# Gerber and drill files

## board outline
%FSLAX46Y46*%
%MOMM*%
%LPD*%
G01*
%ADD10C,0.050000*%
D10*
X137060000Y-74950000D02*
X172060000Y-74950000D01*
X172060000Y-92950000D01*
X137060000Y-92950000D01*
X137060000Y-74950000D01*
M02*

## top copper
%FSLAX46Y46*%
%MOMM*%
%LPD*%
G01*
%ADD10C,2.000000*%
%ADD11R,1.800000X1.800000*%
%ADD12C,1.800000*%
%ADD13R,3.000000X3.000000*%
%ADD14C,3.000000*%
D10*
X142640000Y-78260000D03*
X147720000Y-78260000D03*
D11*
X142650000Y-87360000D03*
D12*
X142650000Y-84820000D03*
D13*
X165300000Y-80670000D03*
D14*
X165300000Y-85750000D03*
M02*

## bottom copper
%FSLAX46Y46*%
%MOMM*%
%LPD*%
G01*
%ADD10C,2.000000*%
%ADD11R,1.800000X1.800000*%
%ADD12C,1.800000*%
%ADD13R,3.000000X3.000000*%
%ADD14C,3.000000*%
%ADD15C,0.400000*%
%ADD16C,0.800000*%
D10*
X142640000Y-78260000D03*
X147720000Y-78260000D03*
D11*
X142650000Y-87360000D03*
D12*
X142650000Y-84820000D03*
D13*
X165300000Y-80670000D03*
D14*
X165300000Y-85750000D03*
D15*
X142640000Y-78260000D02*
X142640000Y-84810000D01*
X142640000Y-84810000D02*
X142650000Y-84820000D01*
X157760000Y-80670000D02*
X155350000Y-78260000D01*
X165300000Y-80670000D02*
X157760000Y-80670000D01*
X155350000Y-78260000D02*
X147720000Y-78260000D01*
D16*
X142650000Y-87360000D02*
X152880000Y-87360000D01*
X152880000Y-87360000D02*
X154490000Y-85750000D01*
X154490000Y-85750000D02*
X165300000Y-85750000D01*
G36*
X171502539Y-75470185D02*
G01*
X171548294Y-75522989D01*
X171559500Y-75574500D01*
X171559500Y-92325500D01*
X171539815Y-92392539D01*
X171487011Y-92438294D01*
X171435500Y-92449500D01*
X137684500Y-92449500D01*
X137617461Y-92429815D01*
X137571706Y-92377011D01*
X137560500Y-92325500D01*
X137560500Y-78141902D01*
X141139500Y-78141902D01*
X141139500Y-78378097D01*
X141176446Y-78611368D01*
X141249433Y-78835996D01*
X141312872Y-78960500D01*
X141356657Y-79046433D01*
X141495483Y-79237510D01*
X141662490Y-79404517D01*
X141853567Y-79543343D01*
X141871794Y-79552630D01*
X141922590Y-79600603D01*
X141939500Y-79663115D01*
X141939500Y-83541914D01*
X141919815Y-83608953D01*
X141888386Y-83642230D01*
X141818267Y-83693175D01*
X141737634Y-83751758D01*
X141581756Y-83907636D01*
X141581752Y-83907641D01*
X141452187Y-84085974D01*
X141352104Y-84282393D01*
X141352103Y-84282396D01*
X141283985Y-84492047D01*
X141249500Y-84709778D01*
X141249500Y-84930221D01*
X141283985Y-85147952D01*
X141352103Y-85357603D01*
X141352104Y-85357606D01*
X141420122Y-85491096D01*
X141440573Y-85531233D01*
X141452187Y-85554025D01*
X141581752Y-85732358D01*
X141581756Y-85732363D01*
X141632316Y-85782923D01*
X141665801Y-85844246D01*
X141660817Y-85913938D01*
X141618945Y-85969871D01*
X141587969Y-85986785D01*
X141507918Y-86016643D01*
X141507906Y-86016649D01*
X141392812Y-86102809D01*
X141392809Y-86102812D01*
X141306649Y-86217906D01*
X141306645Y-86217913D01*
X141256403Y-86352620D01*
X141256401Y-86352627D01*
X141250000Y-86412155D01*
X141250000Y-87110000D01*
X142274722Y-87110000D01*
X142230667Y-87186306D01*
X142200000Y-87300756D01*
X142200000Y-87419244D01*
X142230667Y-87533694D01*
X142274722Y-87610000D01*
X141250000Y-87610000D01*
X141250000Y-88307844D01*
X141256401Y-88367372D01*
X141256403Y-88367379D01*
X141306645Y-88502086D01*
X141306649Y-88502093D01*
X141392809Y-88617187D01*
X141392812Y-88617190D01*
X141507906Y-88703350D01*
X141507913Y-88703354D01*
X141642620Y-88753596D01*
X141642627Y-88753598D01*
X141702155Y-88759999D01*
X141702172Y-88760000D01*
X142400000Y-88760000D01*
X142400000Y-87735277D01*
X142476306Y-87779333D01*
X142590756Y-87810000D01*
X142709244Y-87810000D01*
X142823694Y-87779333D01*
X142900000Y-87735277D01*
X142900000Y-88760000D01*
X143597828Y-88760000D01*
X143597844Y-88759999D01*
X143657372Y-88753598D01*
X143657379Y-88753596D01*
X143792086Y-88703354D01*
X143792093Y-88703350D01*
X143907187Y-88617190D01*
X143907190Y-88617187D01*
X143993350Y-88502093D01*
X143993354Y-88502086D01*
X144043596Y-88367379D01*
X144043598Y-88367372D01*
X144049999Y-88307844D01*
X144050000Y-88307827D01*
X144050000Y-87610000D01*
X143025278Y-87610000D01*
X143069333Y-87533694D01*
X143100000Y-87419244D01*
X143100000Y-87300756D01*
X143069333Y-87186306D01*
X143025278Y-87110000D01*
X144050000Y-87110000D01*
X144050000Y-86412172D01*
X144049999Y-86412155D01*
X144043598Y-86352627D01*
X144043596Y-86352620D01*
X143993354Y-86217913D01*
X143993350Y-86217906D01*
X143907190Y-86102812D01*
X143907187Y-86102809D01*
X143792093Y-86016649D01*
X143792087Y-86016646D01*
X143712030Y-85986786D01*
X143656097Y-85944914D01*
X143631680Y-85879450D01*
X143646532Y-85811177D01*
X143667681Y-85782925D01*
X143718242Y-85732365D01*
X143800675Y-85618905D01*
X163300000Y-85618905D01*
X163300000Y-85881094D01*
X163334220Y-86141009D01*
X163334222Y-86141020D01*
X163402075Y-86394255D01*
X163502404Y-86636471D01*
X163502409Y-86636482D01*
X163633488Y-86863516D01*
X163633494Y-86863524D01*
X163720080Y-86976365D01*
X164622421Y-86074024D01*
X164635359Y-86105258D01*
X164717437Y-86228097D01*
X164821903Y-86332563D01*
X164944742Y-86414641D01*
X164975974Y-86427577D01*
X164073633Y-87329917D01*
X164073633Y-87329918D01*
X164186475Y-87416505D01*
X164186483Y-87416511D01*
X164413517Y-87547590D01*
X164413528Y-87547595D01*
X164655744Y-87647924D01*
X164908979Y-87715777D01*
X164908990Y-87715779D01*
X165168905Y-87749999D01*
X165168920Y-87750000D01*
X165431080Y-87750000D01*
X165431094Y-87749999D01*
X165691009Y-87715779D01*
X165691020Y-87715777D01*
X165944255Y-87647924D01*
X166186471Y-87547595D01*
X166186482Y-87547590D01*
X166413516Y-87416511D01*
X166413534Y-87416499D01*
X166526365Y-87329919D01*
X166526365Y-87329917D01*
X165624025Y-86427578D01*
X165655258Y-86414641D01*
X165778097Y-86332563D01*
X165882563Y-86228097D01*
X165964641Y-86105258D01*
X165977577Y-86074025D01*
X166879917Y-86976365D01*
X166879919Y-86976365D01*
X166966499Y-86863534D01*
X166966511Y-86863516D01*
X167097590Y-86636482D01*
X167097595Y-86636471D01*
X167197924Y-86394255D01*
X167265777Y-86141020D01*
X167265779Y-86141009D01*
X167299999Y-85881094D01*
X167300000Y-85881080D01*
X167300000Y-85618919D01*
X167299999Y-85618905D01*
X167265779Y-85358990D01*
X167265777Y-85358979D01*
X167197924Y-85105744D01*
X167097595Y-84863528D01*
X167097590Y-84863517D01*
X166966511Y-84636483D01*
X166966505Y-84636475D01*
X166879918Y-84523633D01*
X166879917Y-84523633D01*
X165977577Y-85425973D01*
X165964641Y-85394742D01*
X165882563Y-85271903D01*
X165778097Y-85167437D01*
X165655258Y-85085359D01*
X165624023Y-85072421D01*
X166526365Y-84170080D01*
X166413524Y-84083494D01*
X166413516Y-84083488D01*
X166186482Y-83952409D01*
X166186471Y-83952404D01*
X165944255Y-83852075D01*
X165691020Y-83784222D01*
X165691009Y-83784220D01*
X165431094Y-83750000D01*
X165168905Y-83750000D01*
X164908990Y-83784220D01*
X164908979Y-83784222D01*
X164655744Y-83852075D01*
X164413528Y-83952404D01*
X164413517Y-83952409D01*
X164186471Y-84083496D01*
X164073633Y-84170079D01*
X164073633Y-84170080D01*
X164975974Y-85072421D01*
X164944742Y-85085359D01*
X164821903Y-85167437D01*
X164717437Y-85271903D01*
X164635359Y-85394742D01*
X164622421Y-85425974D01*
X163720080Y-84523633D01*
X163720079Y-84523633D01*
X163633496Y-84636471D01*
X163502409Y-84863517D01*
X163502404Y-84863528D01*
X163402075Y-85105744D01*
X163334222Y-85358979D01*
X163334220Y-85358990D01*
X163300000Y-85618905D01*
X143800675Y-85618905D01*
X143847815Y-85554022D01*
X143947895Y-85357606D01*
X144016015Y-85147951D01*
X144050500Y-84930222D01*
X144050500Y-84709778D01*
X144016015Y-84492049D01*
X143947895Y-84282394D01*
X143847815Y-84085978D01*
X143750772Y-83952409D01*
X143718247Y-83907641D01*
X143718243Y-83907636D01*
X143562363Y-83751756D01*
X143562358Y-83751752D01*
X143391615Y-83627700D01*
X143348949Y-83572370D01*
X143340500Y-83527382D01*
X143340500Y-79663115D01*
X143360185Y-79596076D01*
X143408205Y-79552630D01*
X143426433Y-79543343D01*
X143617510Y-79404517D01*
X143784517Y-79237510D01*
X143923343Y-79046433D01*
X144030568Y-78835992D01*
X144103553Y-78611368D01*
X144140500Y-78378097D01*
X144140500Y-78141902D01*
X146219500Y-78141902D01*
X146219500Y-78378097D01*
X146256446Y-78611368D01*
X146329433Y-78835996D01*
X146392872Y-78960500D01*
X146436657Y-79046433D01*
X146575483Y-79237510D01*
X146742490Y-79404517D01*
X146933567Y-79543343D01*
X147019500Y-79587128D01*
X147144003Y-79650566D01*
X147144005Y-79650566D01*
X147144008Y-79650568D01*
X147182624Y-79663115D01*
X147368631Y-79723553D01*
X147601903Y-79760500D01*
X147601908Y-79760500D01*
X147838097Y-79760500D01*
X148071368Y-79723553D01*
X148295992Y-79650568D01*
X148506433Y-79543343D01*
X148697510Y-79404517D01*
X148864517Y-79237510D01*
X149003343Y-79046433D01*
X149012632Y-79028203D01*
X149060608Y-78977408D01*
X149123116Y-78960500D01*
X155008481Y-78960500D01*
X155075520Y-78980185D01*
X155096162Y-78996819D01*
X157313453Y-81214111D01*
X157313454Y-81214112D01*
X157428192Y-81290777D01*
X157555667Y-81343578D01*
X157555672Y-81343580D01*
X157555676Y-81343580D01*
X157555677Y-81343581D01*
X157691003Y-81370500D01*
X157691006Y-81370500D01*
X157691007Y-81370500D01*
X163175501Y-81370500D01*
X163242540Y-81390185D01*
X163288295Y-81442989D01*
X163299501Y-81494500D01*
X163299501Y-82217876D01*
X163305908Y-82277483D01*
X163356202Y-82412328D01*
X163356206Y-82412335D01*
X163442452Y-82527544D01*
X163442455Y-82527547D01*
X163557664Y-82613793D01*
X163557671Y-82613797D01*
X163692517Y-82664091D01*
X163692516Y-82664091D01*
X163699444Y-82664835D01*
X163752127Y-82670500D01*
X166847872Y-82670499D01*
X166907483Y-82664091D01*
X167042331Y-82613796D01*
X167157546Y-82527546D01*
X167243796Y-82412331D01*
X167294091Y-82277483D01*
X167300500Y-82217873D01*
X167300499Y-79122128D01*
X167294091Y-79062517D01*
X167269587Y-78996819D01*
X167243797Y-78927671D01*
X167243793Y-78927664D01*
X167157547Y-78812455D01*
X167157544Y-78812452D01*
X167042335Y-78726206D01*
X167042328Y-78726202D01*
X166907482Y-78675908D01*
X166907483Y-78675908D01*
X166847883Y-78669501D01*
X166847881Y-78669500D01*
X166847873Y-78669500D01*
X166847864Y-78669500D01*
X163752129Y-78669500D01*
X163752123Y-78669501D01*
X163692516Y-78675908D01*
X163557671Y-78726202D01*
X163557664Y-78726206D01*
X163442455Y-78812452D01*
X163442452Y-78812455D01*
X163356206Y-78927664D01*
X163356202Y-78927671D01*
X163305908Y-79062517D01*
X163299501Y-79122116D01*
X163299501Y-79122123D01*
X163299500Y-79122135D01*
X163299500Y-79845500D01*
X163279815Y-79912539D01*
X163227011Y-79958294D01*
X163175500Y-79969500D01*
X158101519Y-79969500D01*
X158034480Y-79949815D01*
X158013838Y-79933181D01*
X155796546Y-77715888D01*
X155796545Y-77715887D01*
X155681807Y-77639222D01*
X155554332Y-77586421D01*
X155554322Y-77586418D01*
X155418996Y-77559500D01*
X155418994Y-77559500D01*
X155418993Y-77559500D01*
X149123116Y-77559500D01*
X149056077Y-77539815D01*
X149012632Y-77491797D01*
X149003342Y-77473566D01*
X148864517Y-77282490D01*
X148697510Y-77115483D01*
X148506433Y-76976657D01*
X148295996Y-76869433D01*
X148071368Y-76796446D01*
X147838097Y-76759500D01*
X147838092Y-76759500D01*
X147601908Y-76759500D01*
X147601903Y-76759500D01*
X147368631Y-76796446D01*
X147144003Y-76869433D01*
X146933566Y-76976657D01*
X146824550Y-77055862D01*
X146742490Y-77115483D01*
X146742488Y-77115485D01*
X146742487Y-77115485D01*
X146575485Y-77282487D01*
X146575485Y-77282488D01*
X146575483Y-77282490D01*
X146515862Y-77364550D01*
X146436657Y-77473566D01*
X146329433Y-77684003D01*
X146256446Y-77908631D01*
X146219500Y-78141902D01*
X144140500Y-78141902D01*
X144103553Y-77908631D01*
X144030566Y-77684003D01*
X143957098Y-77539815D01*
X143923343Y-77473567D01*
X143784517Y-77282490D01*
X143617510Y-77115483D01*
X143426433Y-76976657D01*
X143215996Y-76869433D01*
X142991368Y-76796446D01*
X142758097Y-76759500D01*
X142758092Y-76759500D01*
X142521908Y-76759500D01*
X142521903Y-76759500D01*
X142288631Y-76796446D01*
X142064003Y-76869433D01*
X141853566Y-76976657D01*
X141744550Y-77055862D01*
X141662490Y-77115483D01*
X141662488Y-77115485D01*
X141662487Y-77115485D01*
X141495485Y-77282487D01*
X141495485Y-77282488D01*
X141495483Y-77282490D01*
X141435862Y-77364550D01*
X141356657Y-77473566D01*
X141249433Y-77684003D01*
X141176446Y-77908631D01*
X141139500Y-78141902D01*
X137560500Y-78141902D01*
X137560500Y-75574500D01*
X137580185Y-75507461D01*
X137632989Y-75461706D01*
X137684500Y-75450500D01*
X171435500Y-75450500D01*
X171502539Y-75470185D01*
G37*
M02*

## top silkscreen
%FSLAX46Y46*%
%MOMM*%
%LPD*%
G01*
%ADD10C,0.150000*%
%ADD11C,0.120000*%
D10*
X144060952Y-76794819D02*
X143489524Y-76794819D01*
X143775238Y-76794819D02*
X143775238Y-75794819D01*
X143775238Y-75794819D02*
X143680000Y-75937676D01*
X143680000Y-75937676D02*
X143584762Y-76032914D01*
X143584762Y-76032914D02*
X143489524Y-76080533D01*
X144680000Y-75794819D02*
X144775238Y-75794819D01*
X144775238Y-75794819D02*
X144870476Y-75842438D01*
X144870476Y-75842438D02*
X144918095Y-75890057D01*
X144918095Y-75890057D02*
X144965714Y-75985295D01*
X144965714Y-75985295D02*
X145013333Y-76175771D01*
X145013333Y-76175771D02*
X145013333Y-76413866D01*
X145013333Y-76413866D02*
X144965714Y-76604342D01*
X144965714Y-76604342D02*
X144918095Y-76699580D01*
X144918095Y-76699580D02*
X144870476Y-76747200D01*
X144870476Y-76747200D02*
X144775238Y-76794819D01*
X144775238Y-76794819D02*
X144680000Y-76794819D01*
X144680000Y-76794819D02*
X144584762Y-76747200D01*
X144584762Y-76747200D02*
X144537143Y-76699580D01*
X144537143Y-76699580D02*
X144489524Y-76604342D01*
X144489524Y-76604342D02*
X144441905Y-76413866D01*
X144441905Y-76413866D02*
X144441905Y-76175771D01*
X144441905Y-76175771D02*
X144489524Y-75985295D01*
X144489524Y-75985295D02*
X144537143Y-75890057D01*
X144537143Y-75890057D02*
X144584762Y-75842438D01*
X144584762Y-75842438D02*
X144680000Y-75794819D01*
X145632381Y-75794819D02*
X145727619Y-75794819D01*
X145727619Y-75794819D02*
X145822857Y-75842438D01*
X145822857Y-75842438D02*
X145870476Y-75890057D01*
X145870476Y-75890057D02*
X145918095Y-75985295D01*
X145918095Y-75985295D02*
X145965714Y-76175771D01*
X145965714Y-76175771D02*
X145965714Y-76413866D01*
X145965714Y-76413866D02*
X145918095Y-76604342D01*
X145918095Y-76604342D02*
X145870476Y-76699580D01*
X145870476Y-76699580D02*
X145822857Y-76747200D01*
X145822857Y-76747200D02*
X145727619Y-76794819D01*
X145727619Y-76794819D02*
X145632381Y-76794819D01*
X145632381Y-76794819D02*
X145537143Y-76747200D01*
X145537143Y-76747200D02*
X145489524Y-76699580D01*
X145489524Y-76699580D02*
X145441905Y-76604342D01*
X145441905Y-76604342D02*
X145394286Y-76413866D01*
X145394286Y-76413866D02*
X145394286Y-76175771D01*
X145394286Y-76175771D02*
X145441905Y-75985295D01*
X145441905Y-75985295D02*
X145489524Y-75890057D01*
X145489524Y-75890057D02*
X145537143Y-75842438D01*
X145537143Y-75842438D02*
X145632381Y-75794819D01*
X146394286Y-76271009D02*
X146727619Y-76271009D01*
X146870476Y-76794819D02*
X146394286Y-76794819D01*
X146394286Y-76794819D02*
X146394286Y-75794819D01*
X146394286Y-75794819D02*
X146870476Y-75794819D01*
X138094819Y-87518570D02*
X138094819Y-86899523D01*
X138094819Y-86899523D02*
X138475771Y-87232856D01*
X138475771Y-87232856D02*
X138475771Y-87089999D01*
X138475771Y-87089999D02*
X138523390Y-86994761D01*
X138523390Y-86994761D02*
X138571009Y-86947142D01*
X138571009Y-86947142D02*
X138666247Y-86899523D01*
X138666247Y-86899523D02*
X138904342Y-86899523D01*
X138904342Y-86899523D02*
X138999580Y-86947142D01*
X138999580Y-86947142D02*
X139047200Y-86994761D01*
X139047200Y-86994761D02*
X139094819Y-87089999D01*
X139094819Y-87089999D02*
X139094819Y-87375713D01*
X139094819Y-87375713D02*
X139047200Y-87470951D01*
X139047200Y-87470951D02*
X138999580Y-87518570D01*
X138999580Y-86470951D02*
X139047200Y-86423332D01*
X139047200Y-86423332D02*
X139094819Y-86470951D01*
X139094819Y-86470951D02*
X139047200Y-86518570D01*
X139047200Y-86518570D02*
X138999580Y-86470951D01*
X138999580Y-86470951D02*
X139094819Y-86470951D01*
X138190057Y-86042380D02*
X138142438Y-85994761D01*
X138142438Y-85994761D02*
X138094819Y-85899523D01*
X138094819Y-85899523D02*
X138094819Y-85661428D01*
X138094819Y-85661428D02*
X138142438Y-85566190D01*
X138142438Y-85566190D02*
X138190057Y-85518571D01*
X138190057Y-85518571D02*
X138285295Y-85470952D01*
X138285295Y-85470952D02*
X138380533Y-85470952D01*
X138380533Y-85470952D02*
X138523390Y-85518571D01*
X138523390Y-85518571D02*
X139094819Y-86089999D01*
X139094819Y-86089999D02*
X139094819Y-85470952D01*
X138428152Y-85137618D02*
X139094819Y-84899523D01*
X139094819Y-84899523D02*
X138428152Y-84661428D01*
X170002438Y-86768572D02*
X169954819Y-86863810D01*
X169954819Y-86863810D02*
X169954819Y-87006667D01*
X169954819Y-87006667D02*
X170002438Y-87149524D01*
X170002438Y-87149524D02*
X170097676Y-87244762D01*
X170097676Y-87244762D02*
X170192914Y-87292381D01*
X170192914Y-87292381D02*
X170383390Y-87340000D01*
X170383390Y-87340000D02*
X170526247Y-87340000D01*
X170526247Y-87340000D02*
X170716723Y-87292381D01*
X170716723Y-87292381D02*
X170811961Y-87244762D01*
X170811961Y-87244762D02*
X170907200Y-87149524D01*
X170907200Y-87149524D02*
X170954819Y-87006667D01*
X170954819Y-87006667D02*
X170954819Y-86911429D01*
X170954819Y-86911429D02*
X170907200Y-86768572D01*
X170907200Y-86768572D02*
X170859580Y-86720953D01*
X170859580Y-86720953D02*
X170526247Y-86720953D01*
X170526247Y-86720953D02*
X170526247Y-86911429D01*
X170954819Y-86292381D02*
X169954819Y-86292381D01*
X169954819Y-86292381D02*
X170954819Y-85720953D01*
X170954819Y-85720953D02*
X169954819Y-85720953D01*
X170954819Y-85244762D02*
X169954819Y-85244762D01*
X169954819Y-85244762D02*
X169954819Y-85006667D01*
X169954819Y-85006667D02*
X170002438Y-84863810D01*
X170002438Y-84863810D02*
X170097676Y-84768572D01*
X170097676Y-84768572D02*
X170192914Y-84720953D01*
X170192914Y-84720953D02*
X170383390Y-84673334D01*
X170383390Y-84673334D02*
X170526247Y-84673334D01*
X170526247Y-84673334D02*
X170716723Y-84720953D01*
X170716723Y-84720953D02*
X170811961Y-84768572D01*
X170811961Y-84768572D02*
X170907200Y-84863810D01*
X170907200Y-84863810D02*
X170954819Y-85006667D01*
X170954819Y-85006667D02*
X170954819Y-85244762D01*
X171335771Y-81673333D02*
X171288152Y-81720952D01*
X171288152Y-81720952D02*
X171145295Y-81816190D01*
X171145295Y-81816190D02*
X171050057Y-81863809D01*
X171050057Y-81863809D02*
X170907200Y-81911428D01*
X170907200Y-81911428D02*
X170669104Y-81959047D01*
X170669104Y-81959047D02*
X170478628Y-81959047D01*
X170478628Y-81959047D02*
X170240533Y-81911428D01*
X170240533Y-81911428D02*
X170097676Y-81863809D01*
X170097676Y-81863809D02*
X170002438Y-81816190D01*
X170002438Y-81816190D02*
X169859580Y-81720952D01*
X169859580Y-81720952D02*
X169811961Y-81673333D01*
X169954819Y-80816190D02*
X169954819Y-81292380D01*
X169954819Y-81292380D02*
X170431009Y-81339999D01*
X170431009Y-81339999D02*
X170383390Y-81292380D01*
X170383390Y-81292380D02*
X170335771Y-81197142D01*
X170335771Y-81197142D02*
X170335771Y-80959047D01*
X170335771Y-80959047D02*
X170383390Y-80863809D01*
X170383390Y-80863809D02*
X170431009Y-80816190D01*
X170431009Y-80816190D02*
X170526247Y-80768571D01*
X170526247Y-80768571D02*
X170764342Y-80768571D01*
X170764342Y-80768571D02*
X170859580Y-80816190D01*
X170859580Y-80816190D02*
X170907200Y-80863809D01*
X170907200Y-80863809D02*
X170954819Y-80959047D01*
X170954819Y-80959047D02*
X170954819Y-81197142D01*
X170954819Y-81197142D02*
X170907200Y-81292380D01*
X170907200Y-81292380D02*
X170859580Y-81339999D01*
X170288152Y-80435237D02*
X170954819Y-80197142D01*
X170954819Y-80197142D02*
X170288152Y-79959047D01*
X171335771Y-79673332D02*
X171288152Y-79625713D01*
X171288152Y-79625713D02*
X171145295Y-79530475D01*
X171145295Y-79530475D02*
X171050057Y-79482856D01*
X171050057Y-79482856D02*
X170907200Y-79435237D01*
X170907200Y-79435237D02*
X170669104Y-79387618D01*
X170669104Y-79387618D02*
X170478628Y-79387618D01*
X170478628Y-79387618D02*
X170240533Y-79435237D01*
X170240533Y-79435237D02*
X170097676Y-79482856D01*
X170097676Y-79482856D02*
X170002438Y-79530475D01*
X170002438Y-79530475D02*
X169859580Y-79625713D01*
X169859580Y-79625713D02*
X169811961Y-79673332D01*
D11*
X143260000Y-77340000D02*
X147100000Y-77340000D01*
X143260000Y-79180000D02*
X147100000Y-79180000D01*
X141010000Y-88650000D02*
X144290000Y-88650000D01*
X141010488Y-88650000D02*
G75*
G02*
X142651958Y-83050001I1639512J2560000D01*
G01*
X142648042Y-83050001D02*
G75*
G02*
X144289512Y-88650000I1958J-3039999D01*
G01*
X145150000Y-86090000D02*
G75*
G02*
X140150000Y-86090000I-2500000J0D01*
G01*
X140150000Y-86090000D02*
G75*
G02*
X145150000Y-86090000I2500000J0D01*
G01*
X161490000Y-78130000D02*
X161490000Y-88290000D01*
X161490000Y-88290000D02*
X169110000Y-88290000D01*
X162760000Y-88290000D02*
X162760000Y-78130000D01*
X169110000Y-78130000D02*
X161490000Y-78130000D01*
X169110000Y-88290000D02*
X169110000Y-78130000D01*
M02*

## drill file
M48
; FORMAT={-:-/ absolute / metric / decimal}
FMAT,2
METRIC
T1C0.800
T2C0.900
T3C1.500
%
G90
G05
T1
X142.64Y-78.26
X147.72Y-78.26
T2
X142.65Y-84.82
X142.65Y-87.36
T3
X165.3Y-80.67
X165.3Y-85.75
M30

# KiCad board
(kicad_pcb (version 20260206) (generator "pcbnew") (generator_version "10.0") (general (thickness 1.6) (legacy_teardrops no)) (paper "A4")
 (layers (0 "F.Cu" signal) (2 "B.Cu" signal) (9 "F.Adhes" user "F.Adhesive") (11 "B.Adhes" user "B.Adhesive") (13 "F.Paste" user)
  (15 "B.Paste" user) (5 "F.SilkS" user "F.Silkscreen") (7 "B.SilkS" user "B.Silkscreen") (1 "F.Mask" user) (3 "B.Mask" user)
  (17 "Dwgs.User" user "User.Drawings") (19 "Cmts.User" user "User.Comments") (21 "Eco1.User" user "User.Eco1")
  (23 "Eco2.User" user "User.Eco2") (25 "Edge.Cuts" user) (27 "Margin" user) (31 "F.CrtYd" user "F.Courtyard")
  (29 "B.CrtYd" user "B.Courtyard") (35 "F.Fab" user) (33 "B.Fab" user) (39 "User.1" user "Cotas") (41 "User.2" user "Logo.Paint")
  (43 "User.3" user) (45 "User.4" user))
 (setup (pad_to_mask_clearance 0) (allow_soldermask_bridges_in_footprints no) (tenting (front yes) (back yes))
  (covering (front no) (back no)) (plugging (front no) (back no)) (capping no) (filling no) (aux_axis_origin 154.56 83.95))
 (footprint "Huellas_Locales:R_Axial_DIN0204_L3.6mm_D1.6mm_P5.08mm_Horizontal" (layer "F.Cu") (at 142.64 78.26)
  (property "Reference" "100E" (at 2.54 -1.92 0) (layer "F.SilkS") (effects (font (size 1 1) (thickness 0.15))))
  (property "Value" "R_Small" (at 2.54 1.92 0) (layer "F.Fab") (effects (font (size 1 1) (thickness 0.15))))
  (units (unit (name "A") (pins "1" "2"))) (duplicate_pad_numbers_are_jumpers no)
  (fp_line (start 0.62 -0.92) (end 4.46 -0.92) (stroke (width 0.12) (type solid)) (layer "F.SilkS"))
  (fp_line (start 0.62 0.92) (end 4.46 0.92) (stroke (width 0.12) (type solid)) (layer "F.SilkS"))
  (pad "1" thru_hole circle (at 0 0) (size 2 2) (drill 0.8) (layers "*.Cu" "*.Mask") (remove_unused_layers no) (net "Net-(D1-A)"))
  (pad "2" thru_hole circle (at 5.08 0) (size 2 2) (drill 0.8) (layers "*.Cu" "*.Mask") (remove_unused_layers no) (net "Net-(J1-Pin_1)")))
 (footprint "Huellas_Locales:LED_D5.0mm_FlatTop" (layer "F.Cu") (at 142.65 87.36 90)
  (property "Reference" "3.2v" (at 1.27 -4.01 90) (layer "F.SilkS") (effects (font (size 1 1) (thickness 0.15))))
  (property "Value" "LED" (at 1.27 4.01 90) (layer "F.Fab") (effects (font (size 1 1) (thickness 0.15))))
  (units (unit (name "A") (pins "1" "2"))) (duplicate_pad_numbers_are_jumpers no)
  (fp_line (start -1.29 -1.64) (end -1.29 1.64) (stroke (width 0.12) (type solid)) (layer "F.SilkS"))
  (fp_arc (start -1.29 -1.639512) (mid 2.125106 -2.917258) (end 4.309999 0.001958) (stroke (width 0.12) (type solid)) (layer "F.SilkS"))
  (fp_arc (start 4.309999 -0.001958) (mid 2.125106 2.917258) (end -1.29 1.639512) (stroke (width 0.12) (type solid)) (layer "F.SilkS"))
  (fp_circle (center 1.27 0) (end 3.77 0) (stroke (width 0.12) (type solid)) (fill no) (layer "F.SilkS"))
  (pad "1" thru_hole rect (at 0 0 90) (size 1.8 1.8) (drill 0.9) (layers "*.Cu" "*.Mask") (remove_unused_layers no) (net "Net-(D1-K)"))
  (pad "2" thru_hole circle (at 2.54 0 90) (size 1.8 1.8) (drill 0.9) (layers "*.Cu" "*.Mask") (remove_unused_layers no) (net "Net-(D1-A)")))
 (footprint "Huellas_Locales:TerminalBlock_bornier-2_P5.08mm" (layer "F.Cu") (at 165.3 80.67 -90)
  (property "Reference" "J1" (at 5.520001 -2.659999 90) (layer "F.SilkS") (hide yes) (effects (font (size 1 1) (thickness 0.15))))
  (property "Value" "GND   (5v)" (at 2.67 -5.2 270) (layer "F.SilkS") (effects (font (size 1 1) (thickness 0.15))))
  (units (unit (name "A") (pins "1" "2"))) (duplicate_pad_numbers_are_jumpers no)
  (fp_line (start -2.54 3.81) (end 7.62 3.81) (stroke (width 0.12) (type solid)) (layer "F.SilkS"))
  (fp_line (start 7.62 3.81) (end 7.62 -3.81) (stroke (width 0.12) (type solid)) (layer "F.SilkS"))
  (fp_line (start 7.62 2.54) (end -2.54 2.54) (stroke (width 0.12) (type solid)) (layer "F.SilkS"))
  (fp_line (start -2.54 -3.81) (end -2.54 3.81) (stroke (width 0.12) (type solid)) (layer "F.SilkS"))
  (fp_line (start 7.62 -3.81) (end -2.54 -3.81) (stroke (width 0.12) (type solid)) (layer "F.SilkS"))
  (pad "1" thru_hole rect (at 0 0 270) (size 3 3) (drill 1.5) (layers "*.Cu" "*.Mask") (remove_unused_layers no) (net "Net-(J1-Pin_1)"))
  (pad "2" thru_hole circle (at 5.08 0 270) (size 3 3) (drill 1.5) (layers "*.Cu" "*.Mask") (remove_unused_layers no) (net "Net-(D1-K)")))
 (gr_rect (start 137.06 74.95) (end 172.06 92.95) (stroke (width 0.05) (type default)) (fill no) (layer "Edge.Cuts"))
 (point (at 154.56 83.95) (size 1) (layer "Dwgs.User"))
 (segment (start 142.64 78.26) (end 142.64 84.81) (width 0.4) (layer "B.Cu") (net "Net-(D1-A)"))
 (segment (start 142.64 84.81) (end 142.65 84.82) (width 0.4) (layer "B.Cu") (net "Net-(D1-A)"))
 (segment (start 157.76 80.67) (end 155.35 78.26) (width 0.4) (layer "B.Cu") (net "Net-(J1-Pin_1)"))
 (segment (start 165.3 80.67) (end 157.76 80.67) (width 0.4) (layer "B.Cu") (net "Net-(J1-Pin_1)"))
 (segment (start 155.35 78.26) (end 147.72 78.26) (width 0.4) (layer "B.Cu") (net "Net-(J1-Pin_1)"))
 (segment (start 142.65 87.36) (end 152.88 87.36) (width 0.8) (layer "B.Cu") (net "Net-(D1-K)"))
 (segment (start 152.88 87.36) (end 154.49 85.75) (width 0.8) (layer "B.Cu") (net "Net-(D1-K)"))
 (segment (start 154.49 85.75) (end 165.3 85.75) (width 0.8) (layer "B.Cu") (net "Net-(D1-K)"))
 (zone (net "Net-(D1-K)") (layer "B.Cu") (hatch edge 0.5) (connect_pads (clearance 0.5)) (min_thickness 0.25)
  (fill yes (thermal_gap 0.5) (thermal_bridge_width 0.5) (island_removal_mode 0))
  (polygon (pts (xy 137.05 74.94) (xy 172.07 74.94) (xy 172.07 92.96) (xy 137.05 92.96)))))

